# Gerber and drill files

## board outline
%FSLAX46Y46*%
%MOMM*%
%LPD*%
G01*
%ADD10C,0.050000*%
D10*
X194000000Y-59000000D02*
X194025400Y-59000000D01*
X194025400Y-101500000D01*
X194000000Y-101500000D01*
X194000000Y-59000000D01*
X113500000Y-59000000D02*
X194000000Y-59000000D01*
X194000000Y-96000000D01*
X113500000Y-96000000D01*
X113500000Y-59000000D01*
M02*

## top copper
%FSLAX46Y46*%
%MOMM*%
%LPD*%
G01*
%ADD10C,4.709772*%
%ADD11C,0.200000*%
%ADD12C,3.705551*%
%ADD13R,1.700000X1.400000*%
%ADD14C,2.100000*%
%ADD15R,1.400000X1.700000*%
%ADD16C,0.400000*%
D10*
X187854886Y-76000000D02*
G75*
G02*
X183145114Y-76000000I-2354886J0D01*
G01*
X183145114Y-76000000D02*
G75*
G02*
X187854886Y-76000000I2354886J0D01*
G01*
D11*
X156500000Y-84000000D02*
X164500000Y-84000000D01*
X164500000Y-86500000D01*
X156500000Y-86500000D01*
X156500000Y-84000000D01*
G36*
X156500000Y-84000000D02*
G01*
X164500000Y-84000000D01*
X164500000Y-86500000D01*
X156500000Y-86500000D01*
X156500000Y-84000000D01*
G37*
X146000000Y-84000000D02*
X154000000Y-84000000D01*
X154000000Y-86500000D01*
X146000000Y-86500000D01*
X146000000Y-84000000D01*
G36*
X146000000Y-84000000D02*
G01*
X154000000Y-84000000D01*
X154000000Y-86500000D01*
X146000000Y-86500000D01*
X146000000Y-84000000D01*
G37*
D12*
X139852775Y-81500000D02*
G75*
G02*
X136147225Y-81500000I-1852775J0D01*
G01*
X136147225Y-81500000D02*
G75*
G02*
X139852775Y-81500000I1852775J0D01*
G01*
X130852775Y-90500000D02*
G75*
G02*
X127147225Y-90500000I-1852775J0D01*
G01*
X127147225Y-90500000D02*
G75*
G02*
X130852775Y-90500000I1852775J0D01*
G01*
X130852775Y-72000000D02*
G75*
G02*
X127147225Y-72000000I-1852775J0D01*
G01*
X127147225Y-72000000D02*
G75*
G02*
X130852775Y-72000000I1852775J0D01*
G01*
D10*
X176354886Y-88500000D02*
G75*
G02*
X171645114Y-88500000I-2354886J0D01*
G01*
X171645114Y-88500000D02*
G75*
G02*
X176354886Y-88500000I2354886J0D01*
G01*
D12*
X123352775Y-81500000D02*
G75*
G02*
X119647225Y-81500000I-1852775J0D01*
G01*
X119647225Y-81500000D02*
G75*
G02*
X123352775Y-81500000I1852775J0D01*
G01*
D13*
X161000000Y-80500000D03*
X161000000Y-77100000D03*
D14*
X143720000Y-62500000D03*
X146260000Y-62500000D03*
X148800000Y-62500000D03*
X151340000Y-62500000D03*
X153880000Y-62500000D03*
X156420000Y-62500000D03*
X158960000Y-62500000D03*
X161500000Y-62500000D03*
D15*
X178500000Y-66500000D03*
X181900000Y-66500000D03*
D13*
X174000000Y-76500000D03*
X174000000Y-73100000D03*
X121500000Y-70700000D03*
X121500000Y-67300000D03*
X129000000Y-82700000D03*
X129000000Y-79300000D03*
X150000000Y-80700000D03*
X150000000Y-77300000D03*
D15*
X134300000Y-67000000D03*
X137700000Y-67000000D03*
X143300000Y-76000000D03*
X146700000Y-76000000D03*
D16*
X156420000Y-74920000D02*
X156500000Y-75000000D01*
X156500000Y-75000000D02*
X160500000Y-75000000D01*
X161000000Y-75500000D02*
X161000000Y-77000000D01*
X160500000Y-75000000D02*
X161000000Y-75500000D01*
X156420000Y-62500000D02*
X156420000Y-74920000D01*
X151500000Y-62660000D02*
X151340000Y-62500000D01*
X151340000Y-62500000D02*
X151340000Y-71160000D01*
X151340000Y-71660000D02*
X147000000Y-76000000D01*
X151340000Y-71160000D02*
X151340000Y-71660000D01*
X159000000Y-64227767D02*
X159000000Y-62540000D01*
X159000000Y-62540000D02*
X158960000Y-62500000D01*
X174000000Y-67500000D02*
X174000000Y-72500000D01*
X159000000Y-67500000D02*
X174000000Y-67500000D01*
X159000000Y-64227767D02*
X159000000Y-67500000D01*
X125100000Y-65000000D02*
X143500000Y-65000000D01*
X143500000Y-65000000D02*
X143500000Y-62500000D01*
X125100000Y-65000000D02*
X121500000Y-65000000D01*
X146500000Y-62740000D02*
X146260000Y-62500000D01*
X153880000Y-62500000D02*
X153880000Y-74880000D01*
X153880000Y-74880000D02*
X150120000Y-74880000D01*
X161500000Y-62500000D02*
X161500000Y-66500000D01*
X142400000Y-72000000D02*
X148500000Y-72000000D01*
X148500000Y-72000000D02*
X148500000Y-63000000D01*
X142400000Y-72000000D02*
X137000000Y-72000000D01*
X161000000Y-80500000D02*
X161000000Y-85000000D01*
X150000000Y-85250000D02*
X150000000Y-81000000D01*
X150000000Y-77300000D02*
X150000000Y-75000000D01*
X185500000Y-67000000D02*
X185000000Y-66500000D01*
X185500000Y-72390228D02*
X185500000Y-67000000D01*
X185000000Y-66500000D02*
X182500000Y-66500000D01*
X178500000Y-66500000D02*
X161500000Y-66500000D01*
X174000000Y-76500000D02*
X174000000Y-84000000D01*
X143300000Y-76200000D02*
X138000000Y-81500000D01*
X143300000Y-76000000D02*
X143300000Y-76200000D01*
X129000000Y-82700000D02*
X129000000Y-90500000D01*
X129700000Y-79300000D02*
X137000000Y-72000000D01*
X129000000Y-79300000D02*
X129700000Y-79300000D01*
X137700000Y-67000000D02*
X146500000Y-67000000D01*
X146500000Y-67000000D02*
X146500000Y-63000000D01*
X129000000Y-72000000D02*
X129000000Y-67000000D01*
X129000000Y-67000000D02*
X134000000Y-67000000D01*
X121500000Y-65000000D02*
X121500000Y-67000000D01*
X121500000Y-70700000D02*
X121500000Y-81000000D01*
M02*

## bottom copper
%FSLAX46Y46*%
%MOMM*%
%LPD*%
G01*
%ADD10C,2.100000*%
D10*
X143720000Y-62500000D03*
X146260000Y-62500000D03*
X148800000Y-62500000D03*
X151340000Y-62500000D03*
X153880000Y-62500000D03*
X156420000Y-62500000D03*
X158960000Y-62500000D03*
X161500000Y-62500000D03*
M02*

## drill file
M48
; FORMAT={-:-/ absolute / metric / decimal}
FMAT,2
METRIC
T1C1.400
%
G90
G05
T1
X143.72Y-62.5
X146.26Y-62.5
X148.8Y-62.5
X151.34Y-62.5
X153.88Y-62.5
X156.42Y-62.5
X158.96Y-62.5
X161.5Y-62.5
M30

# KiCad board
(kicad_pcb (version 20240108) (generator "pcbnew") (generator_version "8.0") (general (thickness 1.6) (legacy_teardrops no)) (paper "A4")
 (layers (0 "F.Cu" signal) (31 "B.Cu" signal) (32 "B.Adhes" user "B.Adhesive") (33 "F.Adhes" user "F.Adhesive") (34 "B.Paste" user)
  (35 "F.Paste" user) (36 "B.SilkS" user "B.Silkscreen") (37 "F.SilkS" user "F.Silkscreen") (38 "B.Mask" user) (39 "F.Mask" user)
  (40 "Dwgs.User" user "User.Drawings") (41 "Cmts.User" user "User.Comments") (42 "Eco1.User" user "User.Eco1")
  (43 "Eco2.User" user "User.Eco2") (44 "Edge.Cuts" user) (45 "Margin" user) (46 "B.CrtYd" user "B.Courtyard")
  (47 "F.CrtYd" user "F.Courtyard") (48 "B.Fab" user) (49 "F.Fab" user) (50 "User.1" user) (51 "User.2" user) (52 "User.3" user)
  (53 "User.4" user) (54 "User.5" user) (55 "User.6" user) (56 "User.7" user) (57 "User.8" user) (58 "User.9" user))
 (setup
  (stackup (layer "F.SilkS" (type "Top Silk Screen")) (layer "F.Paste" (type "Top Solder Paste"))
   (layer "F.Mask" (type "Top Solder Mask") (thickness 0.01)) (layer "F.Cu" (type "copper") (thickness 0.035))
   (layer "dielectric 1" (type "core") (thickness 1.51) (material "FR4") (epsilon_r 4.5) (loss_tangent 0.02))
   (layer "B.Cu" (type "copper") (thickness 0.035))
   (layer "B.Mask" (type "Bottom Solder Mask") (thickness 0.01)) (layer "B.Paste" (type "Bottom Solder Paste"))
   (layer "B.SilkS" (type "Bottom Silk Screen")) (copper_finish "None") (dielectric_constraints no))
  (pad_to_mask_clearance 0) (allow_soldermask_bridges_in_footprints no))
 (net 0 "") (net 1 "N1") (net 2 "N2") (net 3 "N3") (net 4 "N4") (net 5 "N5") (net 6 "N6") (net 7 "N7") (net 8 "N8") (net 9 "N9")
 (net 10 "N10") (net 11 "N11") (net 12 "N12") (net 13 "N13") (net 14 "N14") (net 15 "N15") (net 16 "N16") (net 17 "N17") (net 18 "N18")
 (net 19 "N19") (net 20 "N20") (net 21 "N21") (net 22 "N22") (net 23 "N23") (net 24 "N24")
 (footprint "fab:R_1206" (layer "F.Cu") (at 161 78.8 90)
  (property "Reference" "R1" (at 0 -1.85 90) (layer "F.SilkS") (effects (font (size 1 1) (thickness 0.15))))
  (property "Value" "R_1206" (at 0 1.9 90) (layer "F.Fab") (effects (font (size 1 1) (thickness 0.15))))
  (pad "1" smd rect (at -1.7 0 90) (size 1.4 1.7) (layers "F.Cu" "F.Paste" "F.Mask") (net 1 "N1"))
  (pad "2" smd rect (at 1.7 0 90) (size 1.4 1.7) (layers "F.Cu" "F.Paste" "F.Mask") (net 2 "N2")))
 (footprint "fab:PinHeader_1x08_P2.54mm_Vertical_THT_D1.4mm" (layer "F.Cu") (at 143.72 62.5 90)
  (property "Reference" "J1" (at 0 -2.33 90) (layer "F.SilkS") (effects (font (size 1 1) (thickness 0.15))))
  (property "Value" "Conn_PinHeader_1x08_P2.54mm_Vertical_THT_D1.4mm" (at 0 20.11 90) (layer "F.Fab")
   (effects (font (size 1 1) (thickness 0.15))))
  (pad "1" thru_hole circle (at 0 0 90) (size 2.1 2.1) (drill 1.4) (layers "*.Cu" "*.Mask") (remove_unused_layers no) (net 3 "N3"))
  (pad "2" thru_hole circle (at 0 2.54 90) (size 2.1 2.1) (drill 1.4) (layers "*.Cu" "*.Mask") (remove_unused_layers no) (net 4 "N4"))
  (pad "3" thru_hole circle (at 0 5.08 90) (size 2.1 2.1) (drill 1.4) (layers "*.Cu" "*.Mask") (remove_unused_layers no) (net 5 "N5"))
  (pad "4" thru_hole circle (at 0 7.62 90) (size 2.1 2.1) (drill 1.4) (layers "*.Cu" "*.Mask") (remove_unused_layers no) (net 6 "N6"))
  (pad "5" thru_hole circle (at 0 10.16 90) (size 2.1 2.1) (drill 1.4) (layers "*.Cu" "*.Mask") (remove_unused_layers no) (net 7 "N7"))
  (pad "6" thru_hole circle (at 0 12.7 90) (size 2.1 2.1) (drill 1.4) (layers "*.Cu" "*.Mask") (remove_unused_layers no) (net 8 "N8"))
  (pad "7" thru_hole circle (at 0 15.24 90) (size 2.1 2.1) (drill 1.4) (layers "*.Cu" "*.Mask") (remove_unused_layers no) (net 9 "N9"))
  (pad "8" thru_hole circle (at 0 17.78 90) (size 2.1 2.1) (drill 1.4) (layers "*.Cu" "*.Mask") (remove_unused_layers no) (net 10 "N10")))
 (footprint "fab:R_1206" (layer "F.Cu") (at 180.2 66.5)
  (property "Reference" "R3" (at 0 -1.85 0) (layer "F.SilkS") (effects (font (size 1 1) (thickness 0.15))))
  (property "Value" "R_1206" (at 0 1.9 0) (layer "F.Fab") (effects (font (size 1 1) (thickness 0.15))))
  (pad "1" smd rect (at -1.7 0) (size 1.4 1.7) (layers "F.Cu" "F.Paste" "F.Mask") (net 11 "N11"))
  (pad "2" smd rect (at 1.7 0) (size 1.4 1.7) (layers "F.Cu" "F.Paste" "F.Mask") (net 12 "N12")))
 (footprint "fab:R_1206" (layer "F.Cu") (at 174 74.8 90)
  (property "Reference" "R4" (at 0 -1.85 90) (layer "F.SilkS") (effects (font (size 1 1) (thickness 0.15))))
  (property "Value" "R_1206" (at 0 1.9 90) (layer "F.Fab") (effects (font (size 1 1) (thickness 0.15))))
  (pad "1" smd rect (at -1.7 0 90) (size 1.4 1.7) (layers "F.Cu" "F.Paste" "F.Mask") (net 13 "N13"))
  (pad "2" smd rect (at 1.7 0 90) (size 1.4 1.7) (layers "F.Cu" "F.Paste" "F.Mask") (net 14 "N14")))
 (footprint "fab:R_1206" (layer "F.Cu") (at 121.5 69 90)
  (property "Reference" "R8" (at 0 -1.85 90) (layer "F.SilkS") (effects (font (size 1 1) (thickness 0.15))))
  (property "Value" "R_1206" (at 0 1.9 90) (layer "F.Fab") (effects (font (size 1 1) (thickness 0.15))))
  (pad "1" smd rect (at -1.7 0 90) (size 1.4 1.7) (layers "F.Cu" "F.Paste" "F.Mask") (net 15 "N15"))
  (pad "2" smd rect (at 1.7 0 90) (size 1.4 1.7) (layers "F.Cu" "F.Paste" "F.Mask") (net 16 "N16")))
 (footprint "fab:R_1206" (layer "F.Cu") (at 129 81 90)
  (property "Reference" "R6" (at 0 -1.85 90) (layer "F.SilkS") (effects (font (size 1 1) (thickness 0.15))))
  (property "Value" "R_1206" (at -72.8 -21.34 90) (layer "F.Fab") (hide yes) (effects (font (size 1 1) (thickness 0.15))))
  (pad "1" smd rect (at -1.7 0 90) (size 1.4 1.7) (layers "F.Cu" "F.Paste" "F.Mask") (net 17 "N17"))
  (pad "2" smd rect (at 1.7 0 90) (size 1.4 1.7) (layers "F.Cu" "F.Paste" "F.Mask") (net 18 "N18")))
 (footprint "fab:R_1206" (layer "F.Cu") (at 150 79 90)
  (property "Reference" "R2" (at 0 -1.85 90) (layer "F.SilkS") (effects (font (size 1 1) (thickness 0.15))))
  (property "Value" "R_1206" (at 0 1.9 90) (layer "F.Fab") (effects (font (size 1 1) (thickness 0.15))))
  (pad "1" smd rect (at -1.7 0 90) (size 1.4 1.7) (layers "F.Cu" "F.Paste" "F.Mask") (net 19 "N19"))
  (pad "2" smd rect (at 1.7 0 90) (size 1.4 1.7) (layers "F.Cu" "F.Paste" "F.Mask") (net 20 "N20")))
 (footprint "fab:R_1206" (layer "F.Cu") (at 136 67)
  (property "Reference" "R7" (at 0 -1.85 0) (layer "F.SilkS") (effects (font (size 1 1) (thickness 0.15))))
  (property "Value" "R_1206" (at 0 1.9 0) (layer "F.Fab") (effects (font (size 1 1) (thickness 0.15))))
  (pad "1" smd rect (at -1.7 0) (size 1.4 1.7) (layers "F.Cu" "F.Paste" "F.Mask") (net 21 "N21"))
  (pad "2" smd rect (at 1.7 0) (size 1.4 1.7) (layers "F.Cu" "F.Paste" "F.Mask") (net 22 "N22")))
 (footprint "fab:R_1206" (layer "F.Cu") (at 145 76)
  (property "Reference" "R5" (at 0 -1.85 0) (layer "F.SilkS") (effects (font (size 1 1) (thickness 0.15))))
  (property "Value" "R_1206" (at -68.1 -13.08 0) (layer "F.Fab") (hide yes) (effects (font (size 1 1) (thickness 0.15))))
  (pad "1" smd rect (at -1.7 0) (size 1.4 1.7) (layers "F.Cu" "F.Paste" "F.Mask") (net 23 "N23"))
  (pad "2" smd rect (at 1.7 0) (size 1.4 1.7) (layers "F.Cu" "F.Paste" "F.Mask") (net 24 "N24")))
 (gr_circle (center 185.5 76) (end 190.109772 76) (stroke (width 0.2) (type solid)) (fill solid) (layer "F.Cu") (net 12))
 (gr_rect (start 156.5 84) (end 164.5 86.5) (stroke (width 0.2) (type solid)) (fill solid) (layer "F.Cu") (net 1))
 (gr_rect (start 146 84) (end 154 86.5) (stroke (width 0.2) (type solid)) (fill solid) (layer "F.Cu") (net 19))
 (gr_circle (center 138 81.5) (end 141.605551 81.5) (stroke (width 0.2) (type solid)) (fill solid) (layer "F.Cu") (net 23))
 (gr_circle (center 129 90.5) (end 132.605551 90.5) (stroke (width 0.2) (type solid)) (fill solid) (layer "F.Cu") (net 17))
 (gr_circle (center 129 72) (end 132.605551 72) (stroke (width 0.2) (type solid)) (fill solid) (layer "F.Cu") (net 21))
 (gr_circle (center 174 88.5) (end 178.609772 88.5) (stroke (width 0.2) (type solid)) (fill solid) (layer "F.Cu") (net 13))
 (gr_circle (center 121.5 81.5) (end 125.105551 81.5) (stroke (width 0.2) (type solid)) (fill solid) (layer "F.Cu") (net 15))
 (gr_rect (start 194 59) (end 194.0254 101.5) (stroke (width 0.05) (type default)) (fill none) (layer "Edge.Cuts"))
 (gr_rect (start 113.5 59) (end 194 96) (stroke (width 0.05) (type default)) (fill none) (layer "Edge.Cuts"))
 (segment (start 156.42 74.92) (end 156.5 75) (width 0.4) (layer "F.Cu") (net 8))
 (segment (start 156.5 75) (end 160.5 75) (width 0.4) (layer "F.Cu") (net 8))
 (segment (start 161 75.5) (end 161 77) (width 0.4) (layer "F.Cu") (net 8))
 (segment (start 160.5 75) (end 161 75.5) (width 0.4) (layer "F.Cu") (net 8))
 (segment (start 156.42 62.5) (end 156.42 74.92) (width 0.4) (layer "F.Cu") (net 8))
 (segment (start 151.5 62.66) (end 151.34 62.5) (width 0.4) (layer "F.Cu") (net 6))
 (segment (start 151.34 62.5) (end 151.34 71.16) (width 0.4) (layer "F.Cu") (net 6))
 (segment (start 151.34 71.66) (end 147 76) (width 0.4) (layer "F.Cu") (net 6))
 (segment (start 151.34 71.16) (end 151.34 71.66) (width 0.4) (layer "F.Cu") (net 6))
 (segment (start 159 64.227767) (end 159 62.54) (width 0.4) (layer "F.Cu") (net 9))
 (segment (start 159 62.54) (end 158.96 62.5) (width 0.4) (layer "F.Cu") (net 9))
 (segment (start 174 67.5) (end 174 72.5) (width 0.4) (layer "F.Cu") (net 9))
 (segment (start 159 67.5) (end 174 67.5) (width 0.4) (layer "F.Cu") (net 9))
 (segment (start 159 64.227767) (end 159 67.5) (width 0.4) (layer "F.Cu") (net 9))
 (segment (start 125.1 65) (end 143.5 65) (width 0.4) (layer "F.Cu") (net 3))
 (segment (start 143.5 65) (end 143.5 62.5) (width 0.4) (layer "F.Cu") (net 3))
 (segment (start 125.1 65) (end 121.5 65) (width 0.4) (layer "F.Cu") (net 3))
 (segment (start 146.5 62.74) (end 146.26 62.5) (width 0.4) (layer "F.Cu") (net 4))
 (segment (start 153.88 62.5) (end 153.88 74.88) (width 0.4) (layer "F.Cu") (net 7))
 (segment (start 153.88 74.88) (end 150.12 74.88) (width 0.4) (layer "F.Cu") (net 7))
 (segment (start 161.5 62.5) (end 161.5 66.5) (width 0.4) (layer "F.Cu") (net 10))
 (segment (start 142.4 72) (end 148.5 72) (width 0.4) (layer "F.Cu") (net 5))
 (segment (start 148.5 72) (end 148.5 63) (width 0.4) (layer "F.Cu") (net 5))
 (segment (start 142.4 72) (end 137 72) (width 0.4) (layer "F.Cu") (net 5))
 (segment (start 161 80.5) (end 161 85) (width 0.4) (layer "F.Cu") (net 1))
 (segment (start 150 85.25) (end 150 81) (width 0.4) (layer "F.Cu") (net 19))
 (segment (start 150 77.3) (end 150 75) (width 0.4) (layer "F.Cu") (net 20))
 (segment (start 185.5 67) (end 185 66.5) (width 0.4) (layer "F.Cu") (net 12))
 (segment (start 185.5 72.390228) (end 185.5 67) (width 0.4) (layer "F.Cu") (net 12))
 (segment (start 185 66.5) (end 182.5 66.5) (width 0.4) (layer "F.Cu") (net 12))
 (segment (start 178.5 66.5) (end 161.5 66.5) (width 0.4) (layer "F.Cu") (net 11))
 (segment (start 174 76.5) (end 174 84) (width 0.4) (layer "F.Cu") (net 13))
 (segment (start 143.3 76.2) (end 138 81.5) (width 0.4) (layer "F.Cu") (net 23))
 (segment (start 143.3 76) (end 143.3 76.2) (width 0.4) (layer "F.Cu") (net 23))
 (segment (start 129 82.7) (end 129 90.5) (width 0.4) (layer "F.Cu") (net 17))
 (segment (start 129.7 79.3) (end 137 72) (width 0.4) (layer "F.Cu") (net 18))
 (segment (start 129 79.3) (end 129.7 79.3) (width 0.4) (layer "F.Cu") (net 18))
 (segment (start 137.7 67) (end 146.5 67) (width 0.4) (layer "F.Cu") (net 22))
 (segment (start 146.5 67) (end 146.5 63) (width 0.4) (layer "F.Cu") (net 22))
 (segment (start 129 72) (end 129 67) (width 0.4) (layer "F.Cu") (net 21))
 (segment (start 129 67) (end 134 67) (width 0.4) (layer "F.Cu") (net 21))
 (segment (start 121.5 65) (end 121.5 67) (width 0.4) (layer "F.Cu") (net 16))
 (segment (start 121.5 70.7) (end 121.5 81) (width 0.4) (layer "F.Cu") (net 15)))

